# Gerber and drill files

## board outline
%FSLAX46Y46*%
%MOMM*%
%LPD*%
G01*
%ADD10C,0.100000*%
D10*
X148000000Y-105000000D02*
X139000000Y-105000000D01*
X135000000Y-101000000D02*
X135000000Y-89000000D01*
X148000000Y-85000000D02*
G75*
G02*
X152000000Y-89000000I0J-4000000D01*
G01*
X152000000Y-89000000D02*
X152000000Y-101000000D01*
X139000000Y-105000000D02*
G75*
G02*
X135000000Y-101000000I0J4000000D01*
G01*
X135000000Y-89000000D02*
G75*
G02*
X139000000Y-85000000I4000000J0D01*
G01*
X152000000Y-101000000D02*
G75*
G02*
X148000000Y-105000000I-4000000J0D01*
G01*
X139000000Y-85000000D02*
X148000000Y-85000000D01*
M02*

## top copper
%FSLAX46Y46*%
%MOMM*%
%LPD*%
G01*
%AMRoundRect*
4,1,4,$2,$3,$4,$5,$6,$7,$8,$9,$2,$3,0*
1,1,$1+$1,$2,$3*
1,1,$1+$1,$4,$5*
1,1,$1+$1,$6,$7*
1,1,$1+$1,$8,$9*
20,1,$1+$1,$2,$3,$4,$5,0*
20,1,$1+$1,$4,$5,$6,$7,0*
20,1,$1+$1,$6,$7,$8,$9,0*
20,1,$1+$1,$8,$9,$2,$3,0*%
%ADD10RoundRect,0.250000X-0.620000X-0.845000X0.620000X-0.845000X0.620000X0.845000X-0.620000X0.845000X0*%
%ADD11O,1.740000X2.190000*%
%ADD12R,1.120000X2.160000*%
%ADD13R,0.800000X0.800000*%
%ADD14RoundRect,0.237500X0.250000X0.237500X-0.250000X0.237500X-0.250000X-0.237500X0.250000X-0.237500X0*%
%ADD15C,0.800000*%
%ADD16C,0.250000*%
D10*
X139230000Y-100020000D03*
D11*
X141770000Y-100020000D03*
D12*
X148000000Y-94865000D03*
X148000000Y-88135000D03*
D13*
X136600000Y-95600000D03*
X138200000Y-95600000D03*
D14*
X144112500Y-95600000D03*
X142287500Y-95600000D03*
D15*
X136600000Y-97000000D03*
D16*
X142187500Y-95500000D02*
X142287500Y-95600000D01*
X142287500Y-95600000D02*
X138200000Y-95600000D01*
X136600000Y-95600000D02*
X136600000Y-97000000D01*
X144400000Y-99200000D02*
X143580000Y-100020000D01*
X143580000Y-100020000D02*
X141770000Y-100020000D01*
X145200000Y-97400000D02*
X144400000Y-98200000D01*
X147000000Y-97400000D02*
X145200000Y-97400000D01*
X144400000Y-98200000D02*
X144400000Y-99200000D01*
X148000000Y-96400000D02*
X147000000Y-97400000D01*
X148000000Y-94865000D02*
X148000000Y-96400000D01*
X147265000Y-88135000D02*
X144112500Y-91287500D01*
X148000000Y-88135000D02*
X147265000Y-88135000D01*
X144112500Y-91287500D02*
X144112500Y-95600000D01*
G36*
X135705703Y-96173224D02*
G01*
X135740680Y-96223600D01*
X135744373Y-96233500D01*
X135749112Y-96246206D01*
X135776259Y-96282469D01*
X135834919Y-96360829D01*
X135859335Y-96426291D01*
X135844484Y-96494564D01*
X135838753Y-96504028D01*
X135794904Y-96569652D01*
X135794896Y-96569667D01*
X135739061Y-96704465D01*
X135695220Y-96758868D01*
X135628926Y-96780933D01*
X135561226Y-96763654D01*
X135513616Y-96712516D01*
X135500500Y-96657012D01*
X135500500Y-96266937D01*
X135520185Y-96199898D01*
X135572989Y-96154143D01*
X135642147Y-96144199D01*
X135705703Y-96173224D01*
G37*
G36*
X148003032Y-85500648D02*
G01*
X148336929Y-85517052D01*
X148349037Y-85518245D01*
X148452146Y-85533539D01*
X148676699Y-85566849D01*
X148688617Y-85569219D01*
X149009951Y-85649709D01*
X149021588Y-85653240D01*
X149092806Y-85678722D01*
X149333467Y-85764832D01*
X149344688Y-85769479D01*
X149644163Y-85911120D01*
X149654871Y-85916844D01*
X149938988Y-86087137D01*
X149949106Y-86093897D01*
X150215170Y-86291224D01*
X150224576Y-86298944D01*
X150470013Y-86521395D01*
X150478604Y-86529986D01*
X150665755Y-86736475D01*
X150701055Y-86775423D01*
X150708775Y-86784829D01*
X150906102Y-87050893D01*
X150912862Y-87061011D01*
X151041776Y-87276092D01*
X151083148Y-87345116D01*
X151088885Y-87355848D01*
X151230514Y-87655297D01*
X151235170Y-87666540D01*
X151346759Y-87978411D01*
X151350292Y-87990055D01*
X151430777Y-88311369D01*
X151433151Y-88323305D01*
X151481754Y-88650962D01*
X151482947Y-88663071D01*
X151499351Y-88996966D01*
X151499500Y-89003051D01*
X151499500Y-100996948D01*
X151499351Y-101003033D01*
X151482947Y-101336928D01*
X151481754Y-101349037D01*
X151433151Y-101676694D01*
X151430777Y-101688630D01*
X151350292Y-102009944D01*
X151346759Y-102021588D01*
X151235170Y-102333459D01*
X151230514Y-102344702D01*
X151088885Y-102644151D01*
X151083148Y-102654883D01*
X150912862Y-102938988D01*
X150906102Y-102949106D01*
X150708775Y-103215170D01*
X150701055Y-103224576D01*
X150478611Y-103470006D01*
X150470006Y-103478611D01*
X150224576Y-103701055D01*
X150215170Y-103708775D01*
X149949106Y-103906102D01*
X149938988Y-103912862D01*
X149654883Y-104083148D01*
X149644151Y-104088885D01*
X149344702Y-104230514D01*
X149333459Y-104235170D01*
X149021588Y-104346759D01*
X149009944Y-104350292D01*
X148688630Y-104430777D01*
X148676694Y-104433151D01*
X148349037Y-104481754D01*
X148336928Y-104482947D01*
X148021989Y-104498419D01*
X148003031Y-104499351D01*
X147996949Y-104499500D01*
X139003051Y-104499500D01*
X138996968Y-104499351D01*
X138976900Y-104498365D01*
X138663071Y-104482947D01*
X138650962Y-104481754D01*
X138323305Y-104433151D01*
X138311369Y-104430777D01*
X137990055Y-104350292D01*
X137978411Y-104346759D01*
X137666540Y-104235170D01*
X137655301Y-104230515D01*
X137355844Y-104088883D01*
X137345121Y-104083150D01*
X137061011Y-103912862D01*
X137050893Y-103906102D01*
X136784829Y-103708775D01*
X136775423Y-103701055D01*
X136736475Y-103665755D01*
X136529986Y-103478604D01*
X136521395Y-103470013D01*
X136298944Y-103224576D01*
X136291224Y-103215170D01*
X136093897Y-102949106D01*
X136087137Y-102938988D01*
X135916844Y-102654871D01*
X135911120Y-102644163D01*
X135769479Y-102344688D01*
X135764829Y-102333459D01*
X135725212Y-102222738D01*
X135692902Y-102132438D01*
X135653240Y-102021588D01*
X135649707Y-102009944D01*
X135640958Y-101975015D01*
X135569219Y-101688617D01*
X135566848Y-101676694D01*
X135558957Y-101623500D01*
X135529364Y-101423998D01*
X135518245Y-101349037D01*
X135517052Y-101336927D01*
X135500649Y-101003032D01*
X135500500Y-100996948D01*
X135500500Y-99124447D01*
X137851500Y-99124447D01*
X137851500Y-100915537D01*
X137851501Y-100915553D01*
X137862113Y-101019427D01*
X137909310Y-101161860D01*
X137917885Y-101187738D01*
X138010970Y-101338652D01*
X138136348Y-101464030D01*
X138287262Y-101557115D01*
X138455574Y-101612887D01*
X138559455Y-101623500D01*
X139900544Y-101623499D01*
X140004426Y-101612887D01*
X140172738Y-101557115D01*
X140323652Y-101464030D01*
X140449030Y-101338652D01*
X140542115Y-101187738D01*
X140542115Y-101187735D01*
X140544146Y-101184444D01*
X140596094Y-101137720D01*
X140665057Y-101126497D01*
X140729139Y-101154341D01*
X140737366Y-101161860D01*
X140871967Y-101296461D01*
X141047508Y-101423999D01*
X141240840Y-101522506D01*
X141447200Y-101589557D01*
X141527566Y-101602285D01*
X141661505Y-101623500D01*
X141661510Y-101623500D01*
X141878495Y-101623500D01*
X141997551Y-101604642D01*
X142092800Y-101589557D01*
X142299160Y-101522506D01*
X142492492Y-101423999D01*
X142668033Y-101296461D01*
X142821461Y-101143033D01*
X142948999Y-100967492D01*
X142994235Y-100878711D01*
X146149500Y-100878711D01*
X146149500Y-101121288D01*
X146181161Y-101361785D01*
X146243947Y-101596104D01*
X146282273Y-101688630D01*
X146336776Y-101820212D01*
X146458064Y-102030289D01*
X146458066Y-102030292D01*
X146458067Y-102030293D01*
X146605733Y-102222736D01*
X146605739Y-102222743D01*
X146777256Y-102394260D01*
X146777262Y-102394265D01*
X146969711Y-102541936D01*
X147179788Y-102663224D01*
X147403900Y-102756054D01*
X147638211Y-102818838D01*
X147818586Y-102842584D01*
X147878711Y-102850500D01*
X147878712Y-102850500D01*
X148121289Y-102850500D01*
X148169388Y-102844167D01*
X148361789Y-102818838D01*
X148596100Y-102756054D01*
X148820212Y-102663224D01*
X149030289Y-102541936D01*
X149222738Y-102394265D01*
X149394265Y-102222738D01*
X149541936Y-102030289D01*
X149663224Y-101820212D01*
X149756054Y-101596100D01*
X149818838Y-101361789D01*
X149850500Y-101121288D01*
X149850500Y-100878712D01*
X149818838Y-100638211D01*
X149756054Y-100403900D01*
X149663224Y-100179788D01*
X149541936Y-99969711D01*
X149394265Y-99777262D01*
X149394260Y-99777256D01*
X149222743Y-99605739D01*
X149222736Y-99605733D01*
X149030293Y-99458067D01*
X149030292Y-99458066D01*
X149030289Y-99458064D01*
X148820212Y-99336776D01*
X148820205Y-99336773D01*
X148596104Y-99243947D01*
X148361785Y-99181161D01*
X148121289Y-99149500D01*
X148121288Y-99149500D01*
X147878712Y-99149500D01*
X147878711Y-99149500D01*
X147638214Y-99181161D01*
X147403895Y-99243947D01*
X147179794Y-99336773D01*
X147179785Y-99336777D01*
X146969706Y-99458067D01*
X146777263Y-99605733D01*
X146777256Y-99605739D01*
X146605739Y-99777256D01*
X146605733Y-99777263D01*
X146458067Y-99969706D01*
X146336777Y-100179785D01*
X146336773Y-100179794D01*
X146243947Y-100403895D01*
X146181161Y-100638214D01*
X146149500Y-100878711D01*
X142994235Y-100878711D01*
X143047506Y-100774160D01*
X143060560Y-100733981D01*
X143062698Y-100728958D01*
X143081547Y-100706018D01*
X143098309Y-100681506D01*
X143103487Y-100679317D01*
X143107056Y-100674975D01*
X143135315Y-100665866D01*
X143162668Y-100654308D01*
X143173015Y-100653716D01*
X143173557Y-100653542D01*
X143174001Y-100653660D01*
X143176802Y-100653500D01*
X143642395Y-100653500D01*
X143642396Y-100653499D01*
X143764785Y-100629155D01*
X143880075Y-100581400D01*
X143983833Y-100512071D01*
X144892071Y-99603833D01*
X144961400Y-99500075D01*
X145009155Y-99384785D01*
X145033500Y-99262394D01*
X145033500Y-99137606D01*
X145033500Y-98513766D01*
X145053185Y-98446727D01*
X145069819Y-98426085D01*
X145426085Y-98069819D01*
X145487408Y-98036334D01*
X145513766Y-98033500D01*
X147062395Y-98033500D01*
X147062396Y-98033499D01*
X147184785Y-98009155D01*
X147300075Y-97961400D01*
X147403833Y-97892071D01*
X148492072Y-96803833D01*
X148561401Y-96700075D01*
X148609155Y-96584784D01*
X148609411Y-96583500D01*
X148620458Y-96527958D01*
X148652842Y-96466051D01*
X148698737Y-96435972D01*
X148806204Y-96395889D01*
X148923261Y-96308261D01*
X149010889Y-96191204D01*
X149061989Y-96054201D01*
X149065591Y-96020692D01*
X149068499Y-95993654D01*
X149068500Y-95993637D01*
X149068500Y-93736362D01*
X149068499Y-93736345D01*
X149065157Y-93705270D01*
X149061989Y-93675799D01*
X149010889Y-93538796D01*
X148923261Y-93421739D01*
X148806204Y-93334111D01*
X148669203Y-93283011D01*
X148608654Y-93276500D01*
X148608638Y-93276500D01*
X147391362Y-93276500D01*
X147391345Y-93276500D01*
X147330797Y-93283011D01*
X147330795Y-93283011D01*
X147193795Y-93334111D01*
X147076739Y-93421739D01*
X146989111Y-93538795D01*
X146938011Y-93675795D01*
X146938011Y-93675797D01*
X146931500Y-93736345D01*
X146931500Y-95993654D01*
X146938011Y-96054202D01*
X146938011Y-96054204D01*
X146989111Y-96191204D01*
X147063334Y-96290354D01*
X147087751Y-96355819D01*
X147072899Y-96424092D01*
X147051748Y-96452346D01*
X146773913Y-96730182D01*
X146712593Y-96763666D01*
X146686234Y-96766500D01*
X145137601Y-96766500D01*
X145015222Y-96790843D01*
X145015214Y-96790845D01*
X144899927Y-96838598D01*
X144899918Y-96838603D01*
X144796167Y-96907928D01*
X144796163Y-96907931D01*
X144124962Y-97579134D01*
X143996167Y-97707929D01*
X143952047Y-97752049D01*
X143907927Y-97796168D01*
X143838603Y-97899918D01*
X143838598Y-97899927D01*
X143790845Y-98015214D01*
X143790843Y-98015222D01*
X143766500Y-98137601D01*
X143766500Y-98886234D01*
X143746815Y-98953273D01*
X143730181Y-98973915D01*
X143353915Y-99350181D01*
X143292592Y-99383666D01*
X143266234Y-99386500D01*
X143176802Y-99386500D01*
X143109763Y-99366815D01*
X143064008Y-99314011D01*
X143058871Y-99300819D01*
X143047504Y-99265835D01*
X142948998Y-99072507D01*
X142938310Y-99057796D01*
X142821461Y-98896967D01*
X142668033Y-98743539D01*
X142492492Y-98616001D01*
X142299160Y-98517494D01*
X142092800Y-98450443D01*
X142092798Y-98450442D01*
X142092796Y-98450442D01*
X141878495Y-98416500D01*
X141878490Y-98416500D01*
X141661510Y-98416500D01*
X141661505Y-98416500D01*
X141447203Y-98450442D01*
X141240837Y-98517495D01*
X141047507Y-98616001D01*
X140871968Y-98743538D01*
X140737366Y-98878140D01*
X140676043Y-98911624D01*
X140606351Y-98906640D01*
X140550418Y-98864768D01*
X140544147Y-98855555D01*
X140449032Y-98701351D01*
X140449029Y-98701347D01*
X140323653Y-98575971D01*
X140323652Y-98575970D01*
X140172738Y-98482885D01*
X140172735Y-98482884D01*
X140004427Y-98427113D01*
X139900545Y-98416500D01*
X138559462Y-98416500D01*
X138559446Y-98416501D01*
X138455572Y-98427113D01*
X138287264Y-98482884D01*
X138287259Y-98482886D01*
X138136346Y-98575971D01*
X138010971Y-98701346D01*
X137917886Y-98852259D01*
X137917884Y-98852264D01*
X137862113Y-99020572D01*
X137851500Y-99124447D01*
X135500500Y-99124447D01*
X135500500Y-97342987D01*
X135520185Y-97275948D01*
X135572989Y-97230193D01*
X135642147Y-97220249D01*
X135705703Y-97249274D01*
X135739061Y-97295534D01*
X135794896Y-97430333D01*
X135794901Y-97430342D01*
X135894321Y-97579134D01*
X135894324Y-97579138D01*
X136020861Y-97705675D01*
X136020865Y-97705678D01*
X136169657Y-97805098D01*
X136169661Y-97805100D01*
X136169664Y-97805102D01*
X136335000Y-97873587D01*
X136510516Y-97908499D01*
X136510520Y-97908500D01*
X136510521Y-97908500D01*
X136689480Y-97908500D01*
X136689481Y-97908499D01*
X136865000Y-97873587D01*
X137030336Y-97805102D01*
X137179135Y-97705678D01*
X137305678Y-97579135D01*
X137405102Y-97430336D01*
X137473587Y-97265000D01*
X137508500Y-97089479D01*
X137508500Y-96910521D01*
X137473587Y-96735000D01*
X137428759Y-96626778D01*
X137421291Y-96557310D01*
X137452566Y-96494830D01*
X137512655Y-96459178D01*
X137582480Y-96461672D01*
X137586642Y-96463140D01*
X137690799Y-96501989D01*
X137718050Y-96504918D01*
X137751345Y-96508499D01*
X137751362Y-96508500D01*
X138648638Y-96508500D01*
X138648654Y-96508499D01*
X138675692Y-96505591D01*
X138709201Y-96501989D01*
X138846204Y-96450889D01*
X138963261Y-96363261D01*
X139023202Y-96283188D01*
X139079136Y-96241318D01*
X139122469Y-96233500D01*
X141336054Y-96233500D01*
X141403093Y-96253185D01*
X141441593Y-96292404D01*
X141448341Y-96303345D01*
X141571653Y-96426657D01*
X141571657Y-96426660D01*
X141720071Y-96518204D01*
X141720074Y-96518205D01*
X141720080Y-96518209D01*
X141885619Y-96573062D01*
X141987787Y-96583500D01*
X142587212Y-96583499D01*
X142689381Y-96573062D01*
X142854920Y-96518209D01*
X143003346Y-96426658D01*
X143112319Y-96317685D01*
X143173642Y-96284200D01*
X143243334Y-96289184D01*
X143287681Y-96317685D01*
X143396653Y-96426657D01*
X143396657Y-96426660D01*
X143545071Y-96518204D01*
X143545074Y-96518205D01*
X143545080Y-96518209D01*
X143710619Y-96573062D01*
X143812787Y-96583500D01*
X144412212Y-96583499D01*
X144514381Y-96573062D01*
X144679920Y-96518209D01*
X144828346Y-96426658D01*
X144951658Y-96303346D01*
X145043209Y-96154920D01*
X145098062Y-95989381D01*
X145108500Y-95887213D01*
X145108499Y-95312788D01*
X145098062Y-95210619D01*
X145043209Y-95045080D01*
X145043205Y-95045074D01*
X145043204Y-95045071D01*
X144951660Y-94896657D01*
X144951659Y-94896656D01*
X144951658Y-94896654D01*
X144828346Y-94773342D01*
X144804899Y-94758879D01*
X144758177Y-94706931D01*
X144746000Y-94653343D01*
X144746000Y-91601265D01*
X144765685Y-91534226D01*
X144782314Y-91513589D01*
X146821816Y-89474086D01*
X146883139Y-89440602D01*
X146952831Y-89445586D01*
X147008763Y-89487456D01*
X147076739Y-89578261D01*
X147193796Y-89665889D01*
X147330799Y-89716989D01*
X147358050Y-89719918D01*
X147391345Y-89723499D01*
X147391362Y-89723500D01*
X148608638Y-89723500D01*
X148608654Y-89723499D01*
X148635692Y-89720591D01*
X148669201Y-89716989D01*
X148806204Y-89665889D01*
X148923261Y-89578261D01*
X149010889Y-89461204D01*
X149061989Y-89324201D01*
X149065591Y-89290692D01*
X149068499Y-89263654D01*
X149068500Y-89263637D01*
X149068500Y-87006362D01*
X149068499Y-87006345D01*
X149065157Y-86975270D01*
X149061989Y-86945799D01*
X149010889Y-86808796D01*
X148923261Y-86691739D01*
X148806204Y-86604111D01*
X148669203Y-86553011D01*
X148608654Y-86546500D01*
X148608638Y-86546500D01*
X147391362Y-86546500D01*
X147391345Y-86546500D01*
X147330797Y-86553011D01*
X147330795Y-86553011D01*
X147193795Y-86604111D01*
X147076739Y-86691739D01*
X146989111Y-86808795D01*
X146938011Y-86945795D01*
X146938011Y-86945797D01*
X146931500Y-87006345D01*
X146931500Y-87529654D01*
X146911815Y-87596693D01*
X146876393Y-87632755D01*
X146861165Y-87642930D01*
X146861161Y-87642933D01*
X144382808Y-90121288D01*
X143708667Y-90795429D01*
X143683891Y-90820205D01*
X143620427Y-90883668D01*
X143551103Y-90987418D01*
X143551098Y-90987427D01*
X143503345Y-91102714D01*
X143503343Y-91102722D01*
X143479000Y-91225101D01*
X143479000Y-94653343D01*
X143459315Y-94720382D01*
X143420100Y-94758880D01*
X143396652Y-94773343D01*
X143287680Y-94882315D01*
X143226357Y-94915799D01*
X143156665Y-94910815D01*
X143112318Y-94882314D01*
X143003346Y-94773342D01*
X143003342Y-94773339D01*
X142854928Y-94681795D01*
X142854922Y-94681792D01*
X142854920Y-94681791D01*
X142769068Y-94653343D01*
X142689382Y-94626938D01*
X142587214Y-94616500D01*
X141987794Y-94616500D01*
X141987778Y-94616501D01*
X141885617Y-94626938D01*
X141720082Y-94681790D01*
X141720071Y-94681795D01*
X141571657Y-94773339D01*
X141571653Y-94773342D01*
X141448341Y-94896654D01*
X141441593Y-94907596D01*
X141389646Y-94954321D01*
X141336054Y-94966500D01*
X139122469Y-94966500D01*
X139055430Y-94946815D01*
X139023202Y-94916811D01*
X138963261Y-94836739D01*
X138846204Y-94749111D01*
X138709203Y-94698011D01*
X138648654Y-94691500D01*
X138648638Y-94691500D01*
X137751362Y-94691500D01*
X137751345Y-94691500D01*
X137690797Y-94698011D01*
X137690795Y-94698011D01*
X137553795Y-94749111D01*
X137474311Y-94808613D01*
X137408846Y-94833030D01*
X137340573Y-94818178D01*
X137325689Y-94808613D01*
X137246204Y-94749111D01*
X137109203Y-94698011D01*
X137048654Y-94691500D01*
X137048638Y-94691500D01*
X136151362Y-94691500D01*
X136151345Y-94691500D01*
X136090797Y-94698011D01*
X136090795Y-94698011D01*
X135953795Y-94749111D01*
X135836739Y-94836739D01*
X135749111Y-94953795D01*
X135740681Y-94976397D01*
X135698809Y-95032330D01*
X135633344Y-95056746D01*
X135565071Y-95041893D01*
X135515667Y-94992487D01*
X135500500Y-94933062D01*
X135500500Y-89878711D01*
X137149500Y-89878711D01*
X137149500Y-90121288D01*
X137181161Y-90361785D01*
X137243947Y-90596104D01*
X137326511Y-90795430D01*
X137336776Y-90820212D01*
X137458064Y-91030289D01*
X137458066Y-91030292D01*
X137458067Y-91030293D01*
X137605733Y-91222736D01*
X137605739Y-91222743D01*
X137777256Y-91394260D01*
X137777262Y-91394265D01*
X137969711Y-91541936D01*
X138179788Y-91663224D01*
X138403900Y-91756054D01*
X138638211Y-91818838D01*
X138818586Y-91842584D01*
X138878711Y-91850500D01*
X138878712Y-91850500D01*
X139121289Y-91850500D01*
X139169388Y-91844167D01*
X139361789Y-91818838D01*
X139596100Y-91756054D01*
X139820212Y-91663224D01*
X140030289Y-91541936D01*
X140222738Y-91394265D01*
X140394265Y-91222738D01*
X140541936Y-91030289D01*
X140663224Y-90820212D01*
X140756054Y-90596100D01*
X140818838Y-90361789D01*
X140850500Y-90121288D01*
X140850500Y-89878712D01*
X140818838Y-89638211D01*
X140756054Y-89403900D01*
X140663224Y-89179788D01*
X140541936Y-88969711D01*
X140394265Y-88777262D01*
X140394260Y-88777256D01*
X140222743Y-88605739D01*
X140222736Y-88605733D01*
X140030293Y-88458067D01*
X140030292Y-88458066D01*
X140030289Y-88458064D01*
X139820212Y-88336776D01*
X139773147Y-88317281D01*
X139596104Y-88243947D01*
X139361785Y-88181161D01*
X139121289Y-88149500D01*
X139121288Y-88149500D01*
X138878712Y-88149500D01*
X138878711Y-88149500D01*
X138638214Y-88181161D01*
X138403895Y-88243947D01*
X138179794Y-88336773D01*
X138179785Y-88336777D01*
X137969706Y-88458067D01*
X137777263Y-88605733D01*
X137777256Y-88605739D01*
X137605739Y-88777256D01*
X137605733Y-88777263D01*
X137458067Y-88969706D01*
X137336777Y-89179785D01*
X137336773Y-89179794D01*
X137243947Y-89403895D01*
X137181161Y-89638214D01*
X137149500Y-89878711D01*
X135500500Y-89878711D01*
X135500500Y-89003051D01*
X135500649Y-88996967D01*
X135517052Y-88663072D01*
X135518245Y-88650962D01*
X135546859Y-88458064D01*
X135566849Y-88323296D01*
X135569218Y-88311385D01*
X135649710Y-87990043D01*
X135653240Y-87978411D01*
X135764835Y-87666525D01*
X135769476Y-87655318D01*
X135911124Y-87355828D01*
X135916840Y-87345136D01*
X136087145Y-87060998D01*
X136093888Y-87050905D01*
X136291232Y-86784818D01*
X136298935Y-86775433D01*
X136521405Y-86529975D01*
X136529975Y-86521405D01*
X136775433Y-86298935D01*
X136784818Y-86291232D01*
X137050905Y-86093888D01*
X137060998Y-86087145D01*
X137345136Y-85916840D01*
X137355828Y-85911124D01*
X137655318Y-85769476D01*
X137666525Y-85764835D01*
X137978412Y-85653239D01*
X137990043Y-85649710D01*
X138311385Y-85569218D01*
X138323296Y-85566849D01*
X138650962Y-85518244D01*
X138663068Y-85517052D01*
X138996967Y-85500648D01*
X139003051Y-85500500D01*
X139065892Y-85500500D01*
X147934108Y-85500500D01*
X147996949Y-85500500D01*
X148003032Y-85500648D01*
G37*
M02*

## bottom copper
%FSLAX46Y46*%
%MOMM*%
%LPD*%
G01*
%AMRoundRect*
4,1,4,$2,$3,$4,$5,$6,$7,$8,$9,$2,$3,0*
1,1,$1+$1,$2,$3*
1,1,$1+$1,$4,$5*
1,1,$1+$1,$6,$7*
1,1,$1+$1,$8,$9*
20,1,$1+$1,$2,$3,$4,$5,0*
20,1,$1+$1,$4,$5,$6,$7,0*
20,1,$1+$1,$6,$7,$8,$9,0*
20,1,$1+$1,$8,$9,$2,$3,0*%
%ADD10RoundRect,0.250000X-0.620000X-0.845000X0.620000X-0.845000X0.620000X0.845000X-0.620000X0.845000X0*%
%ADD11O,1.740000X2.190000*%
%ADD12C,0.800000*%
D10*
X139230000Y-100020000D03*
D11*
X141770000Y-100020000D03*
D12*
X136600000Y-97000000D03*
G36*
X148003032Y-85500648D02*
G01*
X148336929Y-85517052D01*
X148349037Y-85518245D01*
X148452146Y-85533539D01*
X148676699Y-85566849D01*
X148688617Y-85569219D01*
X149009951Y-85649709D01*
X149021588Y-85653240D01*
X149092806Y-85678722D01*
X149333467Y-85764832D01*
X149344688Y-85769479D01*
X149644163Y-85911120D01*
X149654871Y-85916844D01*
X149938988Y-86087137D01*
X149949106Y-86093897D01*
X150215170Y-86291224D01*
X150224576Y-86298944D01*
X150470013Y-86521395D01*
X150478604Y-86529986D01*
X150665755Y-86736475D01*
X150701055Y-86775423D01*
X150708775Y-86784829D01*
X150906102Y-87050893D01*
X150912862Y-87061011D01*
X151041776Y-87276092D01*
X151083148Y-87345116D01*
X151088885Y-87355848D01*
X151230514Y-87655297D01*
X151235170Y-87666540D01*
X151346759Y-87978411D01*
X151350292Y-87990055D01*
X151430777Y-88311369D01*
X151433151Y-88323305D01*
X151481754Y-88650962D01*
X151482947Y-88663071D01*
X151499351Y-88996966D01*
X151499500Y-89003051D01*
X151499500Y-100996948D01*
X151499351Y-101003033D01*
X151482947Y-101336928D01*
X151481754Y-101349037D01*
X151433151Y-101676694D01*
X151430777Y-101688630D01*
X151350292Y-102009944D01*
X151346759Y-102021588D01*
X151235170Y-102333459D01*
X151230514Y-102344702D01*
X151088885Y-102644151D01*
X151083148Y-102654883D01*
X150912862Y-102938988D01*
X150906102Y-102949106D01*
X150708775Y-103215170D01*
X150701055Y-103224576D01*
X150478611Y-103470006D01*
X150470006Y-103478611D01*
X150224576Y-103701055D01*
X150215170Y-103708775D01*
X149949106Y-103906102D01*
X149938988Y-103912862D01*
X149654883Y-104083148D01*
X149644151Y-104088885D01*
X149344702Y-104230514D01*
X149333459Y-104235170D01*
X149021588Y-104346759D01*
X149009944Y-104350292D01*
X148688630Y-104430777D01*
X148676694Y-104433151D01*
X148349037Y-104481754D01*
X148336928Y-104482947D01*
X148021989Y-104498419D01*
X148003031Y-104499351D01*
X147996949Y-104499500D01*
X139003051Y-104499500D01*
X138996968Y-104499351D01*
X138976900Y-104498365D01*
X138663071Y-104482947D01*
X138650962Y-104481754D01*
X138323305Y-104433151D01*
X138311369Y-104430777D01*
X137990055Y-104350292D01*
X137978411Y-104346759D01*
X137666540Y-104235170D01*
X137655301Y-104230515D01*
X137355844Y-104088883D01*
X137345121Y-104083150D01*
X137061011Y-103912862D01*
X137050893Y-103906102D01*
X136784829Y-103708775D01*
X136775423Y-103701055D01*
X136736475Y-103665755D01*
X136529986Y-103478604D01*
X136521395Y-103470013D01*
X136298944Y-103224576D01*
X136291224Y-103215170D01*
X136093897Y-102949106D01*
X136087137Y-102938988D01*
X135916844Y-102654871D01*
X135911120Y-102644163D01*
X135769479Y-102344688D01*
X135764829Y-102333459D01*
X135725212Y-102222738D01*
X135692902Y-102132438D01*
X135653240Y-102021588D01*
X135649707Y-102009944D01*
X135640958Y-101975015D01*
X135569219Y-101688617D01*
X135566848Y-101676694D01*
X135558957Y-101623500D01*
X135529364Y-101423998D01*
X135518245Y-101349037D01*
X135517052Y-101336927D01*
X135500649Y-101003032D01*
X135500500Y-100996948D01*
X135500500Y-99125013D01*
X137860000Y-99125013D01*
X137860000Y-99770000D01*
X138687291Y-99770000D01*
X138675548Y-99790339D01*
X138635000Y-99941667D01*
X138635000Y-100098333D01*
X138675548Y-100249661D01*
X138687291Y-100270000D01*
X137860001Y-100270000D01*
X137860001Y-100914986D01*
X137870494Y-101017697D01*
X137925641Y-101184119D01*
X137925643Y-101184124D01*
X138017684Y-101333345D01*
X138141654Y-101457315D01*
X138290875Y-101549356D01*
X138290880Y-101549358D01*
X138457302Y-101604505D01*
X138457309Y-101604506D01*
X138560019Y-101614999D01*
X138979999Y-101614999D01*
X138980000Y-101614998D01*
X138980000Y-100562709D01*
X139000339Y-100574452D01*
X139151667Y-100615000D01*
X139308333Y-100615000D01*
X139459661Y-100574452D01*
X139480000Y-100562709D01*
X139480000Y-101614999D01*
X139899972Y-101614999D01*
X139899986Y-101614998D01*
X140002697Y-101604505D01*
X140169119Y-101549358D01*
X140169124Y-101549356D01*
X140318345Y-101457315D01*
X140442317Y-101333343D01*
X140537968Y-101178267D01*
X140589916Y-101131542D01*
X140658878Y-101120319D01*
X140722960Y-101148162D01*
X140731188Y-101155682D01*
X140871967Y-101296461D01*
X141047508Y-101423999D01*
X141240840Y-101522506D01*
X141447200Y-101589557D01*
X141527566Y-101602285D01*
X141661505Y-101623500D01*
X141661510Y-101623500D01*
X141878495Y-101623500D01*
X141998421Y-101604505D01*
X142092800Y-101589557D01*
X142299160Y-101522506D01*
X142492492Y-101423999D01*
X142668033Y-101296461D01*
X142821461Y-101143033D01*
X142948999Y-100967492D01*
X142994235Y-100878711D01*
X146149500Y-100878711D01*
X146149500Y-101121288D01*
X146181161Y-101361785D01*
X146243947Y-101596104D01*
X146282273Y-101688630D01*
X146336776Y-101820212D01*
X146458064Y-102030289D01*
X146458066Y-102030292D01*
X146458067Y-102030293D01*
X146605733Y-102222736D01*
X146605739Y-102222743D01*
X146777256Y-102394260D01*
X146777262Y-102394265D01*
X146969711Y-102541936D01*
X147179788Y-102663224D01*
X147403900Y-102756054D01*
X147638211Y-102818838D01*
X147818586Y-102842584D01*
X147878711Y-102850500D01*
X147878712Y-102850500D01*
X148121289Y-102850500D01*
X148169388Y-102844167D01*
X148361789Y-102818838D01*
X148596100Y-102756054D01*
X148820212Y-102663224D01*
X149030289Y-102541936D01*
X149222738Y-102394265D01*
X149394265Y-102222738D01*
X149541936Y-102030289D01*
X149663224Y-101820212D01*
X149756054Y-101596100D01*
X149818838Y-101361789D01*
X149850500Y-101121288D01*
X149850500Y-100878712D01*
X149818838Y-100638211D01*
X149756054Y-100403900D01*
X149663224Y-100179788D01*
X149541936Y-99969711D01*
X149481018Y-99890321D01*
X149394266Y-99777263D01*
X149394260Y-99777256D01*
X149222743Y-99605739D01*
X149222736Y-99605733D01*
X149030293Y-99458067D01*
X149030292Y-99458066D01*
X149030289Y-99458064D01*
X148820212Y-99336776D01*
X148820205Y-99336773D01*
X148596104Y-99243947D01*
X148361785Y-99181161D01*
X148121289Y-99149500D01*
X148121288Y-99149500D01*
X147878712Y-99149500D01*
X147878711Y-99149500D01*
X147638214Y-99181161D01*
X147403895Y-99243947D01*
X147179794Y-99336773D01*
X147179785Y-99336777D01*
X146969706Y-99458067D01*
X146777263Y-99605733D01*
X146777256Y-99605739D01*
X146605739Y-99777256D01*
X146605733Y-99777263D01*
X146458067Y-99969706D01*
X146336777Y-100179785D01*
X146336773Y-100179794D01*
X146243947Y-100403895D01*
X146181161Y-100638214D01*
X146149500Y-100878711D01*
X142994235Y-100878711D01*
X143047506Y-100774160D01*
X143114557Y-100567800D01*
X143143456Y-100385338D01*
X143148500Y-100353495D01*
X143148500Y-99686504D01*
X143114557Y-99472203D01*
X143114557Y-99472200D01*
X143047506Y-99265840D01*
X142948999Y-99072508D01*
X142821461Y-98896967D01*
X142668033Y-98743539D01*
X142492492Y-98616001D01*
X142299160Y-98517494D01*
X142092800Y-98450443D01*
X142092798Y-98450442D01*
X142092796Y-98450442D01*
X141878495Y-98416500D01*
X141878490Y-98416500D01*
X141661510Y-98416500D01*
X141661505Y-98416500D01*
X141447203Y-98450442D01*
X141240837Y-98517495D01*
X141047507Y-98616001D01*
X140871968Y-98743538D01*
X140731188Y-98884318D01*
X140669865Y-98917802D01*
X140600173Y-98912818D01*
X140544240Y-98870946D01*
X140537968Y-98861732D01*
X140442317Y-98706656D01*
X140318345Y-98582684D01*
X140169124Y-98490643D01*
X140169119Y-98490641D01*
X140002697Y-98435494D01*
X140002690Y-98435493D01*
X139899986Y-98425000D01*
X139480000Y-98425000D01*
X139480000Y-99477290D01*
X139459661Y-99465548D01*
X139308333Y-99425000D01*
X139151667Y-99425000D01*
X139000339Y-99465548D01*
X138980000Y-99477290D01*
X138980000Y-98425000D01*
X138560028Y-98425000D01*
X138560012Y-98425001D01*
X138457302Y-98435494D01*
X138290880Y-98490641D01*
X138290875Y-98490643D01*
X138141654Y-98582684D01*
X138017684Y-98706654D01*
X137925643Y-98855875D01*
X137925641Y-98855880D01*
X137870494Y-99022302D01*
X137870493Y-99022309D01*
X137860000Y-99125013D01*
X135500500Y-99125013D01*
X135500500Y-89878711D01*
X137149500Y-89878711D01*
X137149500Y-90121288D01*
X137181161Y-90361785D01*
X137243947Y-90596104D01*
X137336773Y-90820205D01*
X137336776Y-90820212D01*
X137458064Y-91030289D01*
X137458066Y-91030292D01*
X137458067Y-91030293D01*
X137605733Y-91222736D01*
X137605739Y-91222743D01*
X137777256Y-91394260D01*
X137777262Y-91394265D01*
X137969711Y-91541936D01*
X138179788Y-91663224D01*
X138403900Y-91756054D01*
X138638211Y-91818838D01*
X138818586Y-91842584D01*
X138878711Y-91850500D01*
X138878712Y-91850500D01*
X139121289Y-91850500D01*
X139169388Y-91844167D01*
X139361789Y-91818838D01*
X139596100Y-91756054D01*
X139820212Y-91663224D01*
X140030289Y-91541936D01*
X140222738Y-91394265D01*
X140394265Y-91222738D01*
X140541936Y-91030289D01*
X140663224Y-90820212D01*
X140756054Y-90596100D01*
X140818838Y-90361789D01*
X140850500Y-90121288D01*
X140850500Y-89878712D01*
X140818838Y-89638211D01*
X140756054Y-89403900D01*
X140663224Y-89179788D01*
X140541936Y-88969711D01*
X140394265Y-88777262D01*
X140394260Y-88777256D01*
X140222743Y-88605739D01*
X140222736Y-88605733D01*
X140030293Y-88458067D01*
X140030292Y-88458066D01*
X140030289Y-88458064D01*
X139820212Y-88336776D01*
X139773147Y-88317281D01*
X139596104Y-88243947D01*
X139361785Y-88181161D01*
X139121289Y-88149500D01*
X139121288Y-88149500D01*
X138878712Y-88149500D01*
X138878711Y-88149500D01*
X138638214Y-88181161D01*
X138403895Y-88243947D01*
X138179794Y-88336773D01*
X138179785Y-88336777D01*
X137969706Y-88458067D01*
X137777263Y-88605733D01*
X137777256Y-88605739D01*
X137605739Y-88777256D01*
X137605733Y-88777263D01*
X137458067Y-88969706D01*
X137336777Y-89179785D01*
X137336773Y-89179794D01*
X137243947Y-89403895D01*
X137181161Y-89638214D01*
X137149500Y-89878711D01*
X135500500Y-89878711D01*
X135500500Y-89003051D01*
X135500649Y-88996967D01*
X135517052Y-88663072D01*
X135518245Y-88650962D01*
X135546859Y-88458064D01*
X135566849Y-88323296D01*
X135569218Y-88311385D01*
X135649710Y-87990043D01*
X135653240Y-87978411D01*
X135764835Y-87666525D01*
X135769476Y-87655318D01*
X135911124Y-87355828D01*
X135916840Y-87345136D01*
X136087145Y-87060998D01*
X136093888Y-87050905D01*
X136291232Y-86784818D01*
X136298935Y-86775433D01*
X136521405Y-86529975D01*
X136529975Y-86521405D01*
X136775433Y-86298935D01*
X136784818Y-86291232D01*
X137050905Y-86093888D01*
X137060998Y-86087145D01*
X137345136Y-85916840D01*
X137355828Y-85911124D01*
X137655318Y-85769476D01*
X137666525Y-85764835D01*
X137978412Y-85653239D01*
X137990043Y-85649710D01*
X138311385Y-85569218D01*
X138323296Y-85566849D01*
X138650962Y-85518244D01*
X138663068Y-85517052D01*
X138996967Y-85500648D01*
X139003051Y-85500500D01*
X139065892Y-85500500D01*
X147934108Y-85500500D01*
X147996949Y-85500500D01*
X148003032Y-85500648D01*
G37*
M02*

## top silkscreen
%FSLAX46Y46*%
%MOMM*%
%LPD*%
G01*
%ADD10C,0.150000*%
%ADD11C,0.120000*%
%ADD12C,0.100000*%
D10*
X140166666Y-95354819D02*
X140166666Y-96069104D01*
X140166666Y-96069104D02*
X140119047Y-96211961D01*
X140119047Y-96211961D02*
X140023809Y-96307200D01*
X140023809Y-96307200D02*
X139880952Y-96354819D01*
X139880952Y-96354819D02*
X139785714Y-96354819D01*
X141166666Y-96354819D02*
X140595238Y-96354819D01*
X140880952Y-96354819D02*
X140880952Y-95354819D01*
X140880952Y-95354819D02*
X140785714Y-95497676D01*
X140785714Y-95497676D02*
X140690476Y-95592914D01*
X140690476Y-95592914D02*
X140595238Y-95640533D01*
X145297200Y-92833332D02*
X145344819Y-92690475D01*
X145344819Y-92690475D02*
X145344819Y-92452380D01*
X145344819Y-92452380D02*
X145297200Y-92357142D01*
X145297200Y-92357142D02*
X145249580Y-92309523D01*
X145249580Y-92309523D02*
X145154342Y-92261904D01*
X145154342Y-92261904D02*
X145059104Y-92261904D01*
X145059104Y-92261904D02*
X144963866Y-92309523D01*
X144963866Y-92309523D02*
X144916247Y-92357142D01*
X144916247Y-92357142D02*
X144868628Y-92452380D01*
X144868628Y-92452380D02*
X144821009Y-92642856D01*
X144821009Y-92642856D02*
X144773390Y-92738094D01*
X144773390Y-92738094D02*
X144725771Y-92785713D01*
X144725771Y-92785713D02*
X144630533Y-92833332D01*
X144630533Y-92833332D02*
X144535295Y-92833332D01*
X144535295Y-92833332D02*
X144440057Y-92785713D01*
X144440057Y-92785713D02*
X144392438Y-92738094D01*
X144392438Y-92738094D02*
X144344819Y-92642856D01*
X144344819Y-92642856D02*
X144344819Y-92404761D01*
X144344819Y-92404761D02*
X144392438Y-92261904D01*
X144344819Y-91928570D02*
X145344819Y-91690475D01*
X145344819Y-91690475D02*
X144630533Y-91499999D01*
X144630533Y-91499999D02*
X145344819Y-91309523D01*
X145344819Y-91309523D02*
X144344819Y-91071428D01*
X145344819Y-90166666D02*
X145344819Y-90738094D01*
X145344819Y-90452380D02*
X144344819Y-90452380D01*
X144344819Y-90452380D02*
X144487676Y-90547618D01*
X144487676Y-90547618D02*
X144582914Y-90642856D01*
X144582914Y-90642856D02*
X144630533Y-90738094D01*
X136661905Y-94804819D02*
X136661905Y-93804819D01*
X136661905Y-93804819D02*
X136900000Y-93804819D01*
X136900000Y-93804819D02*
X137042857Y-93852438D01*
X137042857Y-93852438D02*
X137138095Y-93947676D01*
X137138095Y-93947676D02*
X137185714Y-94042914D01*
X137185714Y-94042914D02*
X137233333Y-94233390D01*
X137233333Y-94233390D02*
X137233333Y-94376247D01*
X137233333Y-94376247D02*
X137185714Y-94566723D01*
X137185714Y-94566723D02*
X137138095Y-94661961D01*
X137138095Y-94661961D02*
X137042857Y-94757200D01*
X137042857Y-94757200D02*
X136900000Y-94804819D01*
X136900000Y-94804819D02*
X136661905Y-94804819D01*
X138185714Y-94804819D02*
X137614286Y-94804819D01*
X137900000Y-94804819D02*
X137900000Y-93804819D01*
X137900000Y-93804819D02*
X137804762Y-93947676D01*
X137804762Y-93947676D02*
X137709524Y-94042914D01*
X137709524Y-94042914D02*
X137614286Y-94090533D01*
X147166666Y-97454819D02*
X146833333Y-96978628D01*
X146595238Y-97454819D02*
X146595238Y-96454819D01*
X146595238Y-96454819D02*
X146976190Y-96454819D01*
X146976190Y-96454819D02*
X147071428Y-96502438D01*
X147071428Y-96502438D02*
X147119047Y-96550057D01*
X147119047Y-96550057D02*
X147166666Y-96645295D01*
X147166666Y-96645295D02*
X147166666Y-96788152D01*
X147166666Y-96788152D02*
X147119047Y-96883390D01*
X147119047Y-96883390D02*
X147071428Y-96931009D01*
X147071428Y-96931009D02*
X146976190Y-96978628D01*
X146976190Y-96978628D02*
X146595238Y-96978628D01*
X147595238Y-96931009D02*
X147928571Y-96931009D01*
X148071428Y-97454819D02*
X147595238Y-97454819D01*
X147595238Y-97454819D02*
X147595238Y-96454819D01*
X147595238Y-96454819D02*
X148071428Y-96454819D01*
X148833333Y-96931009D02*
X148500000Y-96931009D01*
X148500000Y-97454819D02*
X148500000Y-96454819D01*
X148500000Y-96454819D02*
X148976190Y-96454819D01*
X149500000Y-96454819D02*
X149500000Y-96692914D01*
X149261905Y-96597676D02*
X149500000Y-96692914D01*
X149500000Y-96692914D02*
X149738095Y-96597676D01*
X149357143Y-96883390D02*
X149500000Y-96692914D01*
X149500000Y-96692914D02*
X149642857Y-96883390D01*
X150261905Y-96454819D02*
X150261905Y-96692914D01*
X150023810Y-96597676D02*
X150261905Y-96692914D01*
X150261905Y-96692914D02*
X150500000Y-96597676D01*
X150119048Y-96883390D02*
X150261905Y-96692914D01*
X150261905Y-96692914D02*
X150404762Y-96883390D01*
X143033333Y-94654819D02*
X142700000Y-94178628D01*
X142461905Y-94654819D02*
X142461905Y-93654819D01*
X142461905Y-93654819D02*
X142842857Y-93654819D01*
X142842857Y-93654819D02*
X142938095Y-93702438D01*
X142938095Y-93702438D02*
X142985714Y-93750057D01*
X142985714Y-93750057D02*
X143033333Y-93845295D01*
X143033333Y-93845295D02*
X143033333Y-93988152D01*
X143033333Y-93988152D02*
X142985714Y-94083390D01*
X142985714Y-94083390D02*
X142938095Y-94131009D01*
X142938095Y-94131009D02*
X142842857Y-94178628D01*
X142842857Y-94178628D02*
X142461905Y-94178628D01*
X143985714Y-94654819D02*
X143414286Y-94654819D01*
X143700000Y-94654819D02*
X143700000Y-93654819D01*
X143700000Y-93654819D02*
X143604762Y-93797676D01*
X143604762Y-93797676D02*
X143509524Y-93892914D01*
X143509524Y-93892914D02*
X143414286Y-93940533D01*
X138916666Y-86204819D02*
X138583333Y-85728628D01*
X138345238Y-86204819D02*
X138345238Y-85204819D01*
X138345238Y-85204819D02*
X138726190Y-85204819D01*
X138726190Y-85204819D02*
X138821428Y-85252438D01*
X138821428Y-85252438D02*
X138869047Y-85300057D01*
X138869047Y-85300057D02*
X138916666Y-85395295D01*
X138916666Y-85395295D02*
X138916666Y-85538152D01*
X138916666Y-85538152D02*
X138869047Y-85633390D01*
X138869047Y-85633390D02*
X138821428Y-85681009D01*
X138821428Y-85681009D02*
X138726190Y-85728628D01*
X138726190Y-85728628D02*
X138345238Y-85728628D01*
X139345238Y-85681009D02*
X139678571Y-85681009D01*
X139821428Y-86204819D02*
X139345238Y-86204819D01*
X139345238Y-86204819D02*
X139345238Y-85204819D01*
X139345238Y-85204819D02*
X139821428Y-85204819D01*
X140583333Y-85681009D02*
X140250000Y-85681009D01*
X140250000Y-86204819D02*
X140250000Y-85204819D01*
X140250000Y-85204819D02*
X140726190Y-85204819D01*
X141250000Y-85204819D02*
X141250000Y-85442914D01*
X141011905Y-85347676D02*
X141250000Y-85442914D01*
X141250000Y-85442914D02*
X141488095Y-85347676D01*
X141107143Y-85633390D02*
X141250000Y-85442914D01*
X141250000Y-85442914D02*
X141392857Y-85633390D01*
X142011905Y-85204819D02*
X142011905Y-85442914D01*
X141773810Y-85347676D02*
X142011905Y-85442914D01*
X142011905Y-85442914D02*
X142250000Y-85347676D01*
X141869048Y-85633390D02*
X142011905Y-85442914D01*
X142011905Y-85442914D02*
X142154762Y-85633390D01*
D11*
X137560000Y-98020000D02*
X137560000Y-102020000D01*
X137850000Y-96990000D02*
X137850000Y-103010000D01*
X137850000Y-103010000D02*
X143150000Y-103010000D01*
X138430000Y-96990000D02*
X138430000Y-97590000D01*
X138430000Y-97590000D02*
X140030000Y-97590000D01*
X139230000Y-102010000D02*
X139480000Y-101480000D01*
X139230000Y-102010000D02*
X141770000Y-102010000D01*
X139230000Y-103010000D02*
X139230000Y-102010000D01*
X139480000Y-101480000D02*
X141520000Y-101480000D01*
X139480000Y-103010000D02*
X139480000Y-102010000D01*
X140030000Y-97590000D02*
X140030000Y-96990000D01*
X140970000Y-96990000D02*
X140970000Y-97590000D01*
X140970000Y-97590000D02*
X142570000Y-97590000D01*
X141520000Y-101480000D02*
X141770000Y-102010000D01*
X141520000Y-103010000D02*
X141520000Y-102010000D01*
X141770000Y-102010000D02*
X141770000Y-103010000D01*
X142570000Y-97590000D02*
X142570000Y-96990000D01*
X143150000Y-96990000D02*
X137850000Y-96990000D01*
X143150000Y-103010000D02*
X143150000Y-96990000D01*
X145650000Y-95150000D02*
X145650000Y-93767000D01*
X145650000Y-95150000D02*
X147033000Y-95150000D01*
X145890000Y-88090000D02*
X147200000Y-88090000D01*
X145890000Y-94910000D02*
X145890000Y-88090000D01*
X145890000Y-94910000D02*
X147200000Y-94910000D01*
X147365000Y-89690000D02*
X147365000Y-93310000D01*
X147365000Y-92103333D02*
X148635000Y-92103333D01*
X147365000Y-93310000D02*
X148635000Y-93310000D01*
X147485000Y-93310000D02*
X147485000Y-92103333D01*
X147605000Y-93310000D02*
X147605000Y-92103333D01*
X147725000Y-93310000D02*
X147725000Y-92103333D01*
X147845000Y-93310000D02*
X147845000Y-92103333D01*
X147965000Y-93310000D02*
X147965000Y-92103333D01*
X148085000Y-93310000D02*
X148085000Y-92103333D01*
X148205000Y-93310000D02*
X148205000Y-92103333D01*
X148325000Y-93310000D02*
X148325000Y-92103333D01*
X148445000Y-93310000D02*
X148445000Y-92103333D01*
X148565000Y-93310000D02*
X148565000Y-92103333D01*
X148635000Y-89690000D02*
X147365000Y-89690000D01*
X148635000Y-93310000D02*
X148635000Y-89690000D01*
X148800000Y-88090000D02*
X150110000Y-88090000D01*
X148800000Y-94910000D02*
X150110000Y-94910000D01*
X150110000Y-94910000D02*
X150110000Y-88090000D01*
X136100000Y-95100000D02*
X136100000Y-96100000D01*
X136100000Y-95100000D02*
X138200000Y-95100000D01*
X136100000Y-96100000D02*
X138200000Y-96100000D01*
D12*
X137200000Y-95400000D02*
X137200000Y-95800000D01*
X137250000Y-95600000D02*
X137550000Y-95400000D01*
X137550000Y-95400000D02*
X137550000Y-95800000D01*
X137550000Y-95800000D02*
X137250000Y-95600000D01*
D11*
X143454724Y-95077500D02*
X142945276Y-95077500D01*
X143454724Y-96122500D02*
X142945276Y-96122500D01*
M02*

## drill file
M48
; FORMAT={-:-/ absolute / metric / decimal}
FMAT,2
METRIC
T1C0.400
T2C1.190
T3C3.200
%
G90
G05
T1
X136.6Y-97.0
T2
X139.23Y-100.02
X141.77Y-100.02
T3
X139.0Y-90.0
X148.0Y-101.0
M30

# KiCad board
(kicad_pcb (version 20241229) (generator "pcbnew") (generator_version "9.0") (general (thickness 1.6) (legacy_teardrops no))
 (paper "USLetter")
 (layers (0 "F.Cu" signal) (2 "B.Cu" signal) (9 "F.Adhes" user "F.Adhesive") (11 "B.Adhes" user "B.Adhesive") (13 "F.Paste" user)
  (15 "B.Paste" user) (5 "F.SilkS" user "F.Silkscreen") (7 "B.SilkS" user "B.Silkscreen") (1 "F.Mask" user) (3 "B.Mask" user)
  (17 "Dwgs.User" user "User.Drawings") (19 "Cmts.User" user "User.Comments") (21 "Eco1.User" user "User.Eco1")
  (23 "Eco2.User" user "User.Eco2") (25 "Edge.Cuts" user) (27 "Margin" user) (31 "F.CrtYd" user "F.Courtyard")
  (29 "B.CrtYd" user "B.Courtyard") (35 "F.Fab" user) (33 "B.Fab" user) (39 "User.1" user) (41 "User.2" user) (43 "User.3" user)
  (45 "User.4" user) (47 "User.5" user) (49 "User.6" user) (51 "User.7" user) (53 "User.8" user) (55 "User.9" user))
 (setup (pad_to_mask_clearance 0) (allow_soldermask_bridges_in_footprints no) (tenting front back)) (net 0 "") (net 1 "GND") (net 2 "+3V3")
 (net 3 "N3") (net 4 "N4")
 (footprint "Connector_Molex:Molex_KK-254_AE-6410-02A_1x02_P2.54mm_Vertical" (layer "F.Cu") (at 139.23 100.02)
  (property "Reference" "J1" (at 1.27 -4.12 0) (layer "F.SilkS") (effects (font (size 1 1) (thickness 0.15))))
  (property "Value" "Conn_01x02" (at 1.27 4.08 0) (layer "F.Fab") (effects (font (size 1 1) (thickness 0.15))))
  (fp_line (start -1.67 -2) (end -1.67 2) (stroke (width 0.12) (type solid)) (layer "F.SilkS"))
  (fp_line (start -1.38 -3.03) (end -1.38 2.99) (stroke (width 0.12) (type solid)) (layer "F.SilkS"))
  (fp_line (start -1.38 2.99) (end 3.92 2.99) (stroke (width 0.12) (type solid)) (layer "F.SilkS"))
  (fp_line (start -0.8 -3.03) (end -0.8 -2.43) (stroke (width 0.12) (type solid)) (layer "F.SilkS"))
  (fp_line (start -0.8 -2.43) (end 0.8 -2.43) (stroke (width 0.12) (type solid)) (layer "F.SilkS"))
  (fp_line (start 0 1.99) (end 0.25 1.46) (stroke (width 0.12) (type solid)) (layer "F.SilkS"))
  (fp_line (start 0 1.99) (end 2.54 1.99) (stroke (width 0.12) (type solid)) (layer "F.SilkS"))
  (fp_line (start 0 2.99) (end 0 1.99) (stroke (width 0.12) (type solid)) (layer "F.SilkS"))
  (fp_line (start 0.25 1.46) (end 2.29 1.46) (stroke (width 0.12) (type solid)) (layer "F.SilkS"))
  (fp_line (start 0.25 2.99) (end 0.25 1.99) (stroke (width 0.12) (type solid)) (layer "F.SilkS"))
  (fp_line (start 0.8 -2.43) (end 0.8 -3.03) (stroke (width 0.12) (type solid)) (layer "F.SilkS"))
  (fp_line (start 1.74 -3.03) (end 1.74 -2.43) (stroke (width 0.12) (type solid)) (layer "F.SilkS"))
  (fp_line (start 1.74 -2.43) (end 3.34 -2.43) (stroke (width 0.12) (type solid)) (layer "F.SilkS"))
  (fp_line (start 2.29 1.46) (end 2.54 1.99) (stroke (width 0.12) (type solid)) (layer "F.SilkS"))
  (fp_line (start 2.29 2.99) (end 2.29 1.99) (stroke (width 0.12) (type solid)) (layer "F.SilkS"))
  (fp_line (start 2.54 1.99) (end 2.54 2.99) (stroke (width 0.12) (type solid)) (layer "F.SilkS"))
  (fp_line (start 3.34 -2.43) (end 3.34 -3.03) (stroke (width 0.12) (type solid)) (layer "F.SilkS"))
  (fp_line (start 3.92 -3.03) (end -1.38 -3.03) (stroke (width 0.12) (type solid)) (layer "F.SilkS"))
  (fp_line (start 3.92 2.99) (end 3.92 -3.03) (stroke (width 0.12) (type solid)) (layer "F.SilkS"))
  (pad "1" thru_hole roundrect (at 0 0) (size 1.74 2.19) (drill 1.19) (layers "*.Cu" "*.Mask") (remove_unused_layers no)
   (roundrect_rratio 0.143678) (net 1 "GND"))
  (pad "2" thru_hole oval (at 2.54 0) (size 1.74 2.19) (drill 1.19) (layers "*.Cu" "*.Mask") (remove_unused_layers no) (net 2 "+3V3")))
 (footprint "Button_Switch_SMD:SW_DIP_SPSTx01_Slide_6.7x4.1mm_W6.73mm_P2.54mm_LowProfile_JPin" (layer "F.Cu") (at 148 91.5 90)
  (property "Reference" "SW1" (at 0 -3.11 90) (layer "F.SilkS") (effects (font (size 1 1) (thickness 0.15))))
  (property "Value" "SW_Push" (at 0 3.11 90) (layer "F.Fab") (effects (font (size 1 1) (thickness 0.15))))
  (fp_line (start -3.65 -2.35) (end -2.267 -2.35) (stroke (width 0.12) (type solid)) (layer "F.SilkS"))
  (fp_line (start -3.65 -2.35) (end -3.65 -0.967) (stroke (width 0.12) (type solid)) (layer "F.SilkS"))
  (fp_line (start 3.41 -2.11) (end 3.41 -0.8) (stroke (width 0.12) (type solid)) (layer "F.SilkS"))
  (fp_line (start -3.41 -2.11) (end 3.41 -2.11) (stroke (width 0.12) (type solid)) (layer "F.SilkS"))
  (fp_line (start -3.41 -2.11) (end -3.41 -0.8) (stroke (width 0.12) (type solid)) (layer "F.SilkS"))
  (fp_line (start 1.81 -0.635) (end -1.81 -0.635) (stroke (width 0.12) (type solid)) (layer "F.SilkS"))
  (fp_line (start -0.603333 -0.635) (end -0.603333 0.635) (stroke (width 0.12) (type solid)) (layer "F.SilkS"))
  (fp_line (start -1.81 -0.635) (end -1.81 0.635) (stroke (width 0.12) (type solid)) (layer "F.SilkS"))
  (fp_line (start -1.81 -0.515) (end -0.603333 -0.515) (stroke (width 0.12) (type solid)) (layer "F.SilkS"))
  (fp_line (start -1.81 -0.395) (end -0.603333 -0.395) (stroke (width 0.12) (type solid)) (layer "F.SilkS"))
  (fp_line (start -1.81 -0.275) (end -0.603333 -0.275) (stroke (width 0.12) (type solid)) (layer "F.SilkS"))
  (fp_line (start -1.81 -0.155) (end -0.603333 -0.155) (stroke (width 0.12) (type solid)) (layer "F.SilkS"))
  (fp_line (start -1.81 -0.035) (end -0.603333 -0.035) (stroke (width 0.12) (type solid)) (layer "F.SilkS"))
  (fp_line (start -1.81 0.085) (end -0.603333 0.085) (stroke (width 0.12) (type solid)) (layer "F.SilkS"))
  (fp_line (start -1.81 0.205) (end -0.603333 0.205) (stroke (width 0.12) (type solid)) (layer "F.SilkS"))
  (fp_line (start -1.81 0.325) (end -0.603333 0.325) (stroke (width 0.12) (type solid)) (layer "F.SilkS"))
  (fp_line (start -1.81 0.445) (end -0.603333 0.445) (stroke (width 0.12) (type solid)) (layer "F.SilkS"))
  (fp_line (start -1.81 0.565) (end -0.603333 0.565) (stroke (width 0.12) (type solid)) (layer "F.SilkS"))
  (fp_line (start 1.81 0.635) (end 1.81 -0.635) (stroke (width 0.12) (type solid)) (layer "F.SilkS"))
  (fp_line (start -1.81 0.635) (end 1.81 0.635) (stroke (width 0.12) (type solid)) (layer "F.SilkS"))
  (fp_line (start 3.41 0.8) (end 3.41 2.11) (stroke (width 0.12) (type solid)) (layer "F.SilkS"))
  (fp_line (start -3.41 0.8) (end -3.41 2.11) (stroke (width 0.12) (type solid)) (layer "F.SilkS"))
  (fp_line (start -3.41 2.11) (end 3.41 2.11) (stroke (width 0.12) (type solid)) (layer "F.SilkS"))
  (pad "1" smd rect (at -3.365 0 90) (size 2.16 1.12) (layers "F.Cu" "F.Mask" "F.Paste") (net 2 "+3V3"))
  (pad "2" smd rect (at 3.365 0 90) (size 2.16 1.12) (layers "F.Cu" "F.Mask" "F.Paste") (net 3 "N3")))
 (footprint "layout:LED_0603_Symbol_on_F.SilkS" (layer "F.Cu") (at 137.4 95.6)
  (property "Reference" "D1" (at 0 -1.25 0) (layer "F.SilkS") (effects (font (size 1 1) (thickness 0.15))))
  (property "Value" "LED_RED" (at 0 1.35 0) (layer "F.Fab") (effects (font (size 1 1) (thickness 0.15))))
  (fp_line (start -1.3 -0.5) (end -1.3 0.5) (stroke (width 0.12) (type solid)) (layer "F.SilkS"))
  (fp_line (start -1.3 -0.5) (end 0.8 -0.5) (stroke (width 0.12) (type solid)) (layer "F.SilkS"))
  (fp_line (start -1.3 0.5) (end 0.8 0.5) (stroke (width 0.12) (type solid)) (layer "F.SilkS"))
  (fp_line (start -0.2 -0.2) (end -0.2 0.2) (stroke (width 0.1) (type solid)) (layer "F.SilkS"))
  (fp_line (start -0.15 0) (end 0.15 -0.2) (stroke (width 0.1) (type solid)) (layer "F.SilkS"))
  (fp_line (start 0.15 -0.2) (end 0.15 0.2) (stroke (width 0.1) (type solid)) (layer "F.SilkS"))
  (fp_line (start 0.15 0.2) (end -0.15 0) (stroke (width 0.1) (type solid)) (layer "F.SilkS"))
  (pad "1" smd rect (at -0.8 0 180) (size 0.8 0.8) (layers "F.Cu" "F.Mask" "F.Paste") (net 1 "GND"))
  (pad "2" smd rect (at 0.8 0 180) (size 0.8 0.8) (layers "F.Cu" "F.Mask" "F.Paste") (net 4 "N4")))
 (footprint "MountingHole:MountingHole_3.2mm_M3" (layer "F.Cu") (at 148 101)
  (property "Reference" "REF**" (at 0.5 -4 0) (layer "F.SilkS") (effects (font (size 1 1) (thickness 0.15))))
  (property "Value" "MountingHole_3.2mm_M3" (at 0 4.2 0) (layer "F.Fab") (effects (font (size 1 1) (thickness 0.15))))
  (pad "" np_thru_hole circle (at 0 0) (size 3.2 3.2) (drill 3.2) (layers "*.Cu" "*.Mask")))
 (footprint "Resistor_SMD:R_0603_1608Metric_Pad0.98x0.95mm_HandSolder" (layer "F.Cu") (at 143.2 95.6 180)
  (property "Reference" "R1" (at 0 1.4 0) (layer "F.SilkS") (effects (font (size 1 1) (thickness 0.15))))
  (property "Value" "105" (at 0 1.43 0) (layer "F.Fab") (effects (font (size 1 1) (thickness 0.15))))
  (fp_line (start -0.254724 0.5225) (end 0.254724 0.5225) (stroke (width 0.12) (type solid)) (layer "F.SilkS"))
  (fp_line (start -0.254724 -0.5225) (end 0.254724 -0.5225) (stroke (width 0.12) (type solid)) (layer "F.SilkS"))
  (pad "1" smd roundrect (at -0.9125 0 180) (size 0.975 0.95) (layers "F.Cu" "F.Mask" "F.Paste") (roundrect_rratio 0.25) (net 3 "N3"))
  (pad "2" smd roundrect (at 0.9125 0 180) (size 0.975 0.95) (layers "F.Cu" "F.Mask" "F.Paste") (roundrect_rratio 0.25) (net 4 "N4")))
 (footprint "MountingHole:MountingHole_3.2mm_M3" (layer "F.Cu") (at 139 90)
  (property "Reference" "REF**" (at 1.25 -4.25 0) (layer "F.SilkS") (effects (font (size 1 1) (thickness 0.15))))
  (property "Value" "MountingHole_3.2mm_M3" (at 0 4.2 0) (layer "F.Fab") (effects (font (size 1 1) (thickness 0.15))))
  (pad "" np_thru_hole circle (at 0 0) (size 3.2 3.2) (drill 3.2) (layers "*.Cu" "*.Mask")))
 (gr_line (start 148 105) (end 139 105) (stroke (width 0.1) (type default)) (layer "Edge.Cuts"))
 (gr_line (start 135 101) (end 135 89) (stroke (width 0.1) (type default)) (layer "Edge.Cuts"))
 (gr_arc (start 148 85) (mid 150.828427 86.171573) (end 152 89) (stroke (width 0.1) (type default)) (layer "Edge.Cuts"))
 (gr_line (start 152 89) (end 152 101) (stroke (width 0.1) (type default)) (layer "Edge.Cuts"))
 (gr_arc (start 139 105) (mid 136.171573 103.828427) (end 135 101) (stroke (width 0.1) (type default)) (layer "Edge.Cuts"))
 (gr_arc (start 135 89) (mid 136.171573 86.171573) (end 139 85) (stroke (width 0.1) (type default)) (layer "Edge.Cuts"))
 (gr_arc (start 152 101) (mid 150.828427 103.828427) (end 148 105) (stroke (width 0.1) (type default)) (layer "Edge.Cuts"))
 (gr_line (start 139 85) (end 148 85) (stroke (width 0.1) (type default)) (layer "Edge.Cuts"))
 (segment (start 142.1875 95.5) (end 142.2875 95.6) (width 0.25) (layer "F.Cu") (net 4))
 (segment (start 142.2875 95.6) (end 138.2 95.6) (width 0.25) (layer "F.Cu") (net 4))
 (segment (start 136.6 95.6) (end 136.6 97) (width 0.25) (layer "F.Cu") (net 1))
 (via (at 136.6 97) (size 0.8) (drill 0.4) (layers "F.Cu" "B.Cu") (free yes) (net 1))
 (segment (start 144.4 99.2) (end 143.58 100.02) (width 0.25) (layer "F.Cu") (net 2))
 (segment (start 143.58 100.02) (end 141.77 100.02) (width 0.25) (layer "F.Cu") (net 2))
 (segment (start 145.2 97.4) (end 144.4 98.2) (width 0.25) (layer "F.Cu") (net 2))
 (segment (start 147 97.4) (end 145.2 97.4) (width 0.25) (layer "F.Cu") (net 2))
 (segment (start 144.4 98.2) (end 144.4 99.2) (width 0.25) (layer "F.Cu") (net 2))
 (segment (start 148 96.4) (end 147 97.4) (width 0.25) (layer "F.Cu") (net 2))
 (segment (start 148 94.865) (end 148 96.4) (width 0.25) (layer "F.Cu") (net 2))
 (segment (start 147.265 88.135) (end 144.1125 91.2875) (width 0.25) (layer "F.Cu") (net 3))
 (segment (start 148 88.135) (end 147.265 88.135) (width 0.25) (layer "F.Cu") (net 3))
 (segment (start 144.1125 91.2875) (end 144.1125 95.6) (width 0.25) (layer "F.Cu") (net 3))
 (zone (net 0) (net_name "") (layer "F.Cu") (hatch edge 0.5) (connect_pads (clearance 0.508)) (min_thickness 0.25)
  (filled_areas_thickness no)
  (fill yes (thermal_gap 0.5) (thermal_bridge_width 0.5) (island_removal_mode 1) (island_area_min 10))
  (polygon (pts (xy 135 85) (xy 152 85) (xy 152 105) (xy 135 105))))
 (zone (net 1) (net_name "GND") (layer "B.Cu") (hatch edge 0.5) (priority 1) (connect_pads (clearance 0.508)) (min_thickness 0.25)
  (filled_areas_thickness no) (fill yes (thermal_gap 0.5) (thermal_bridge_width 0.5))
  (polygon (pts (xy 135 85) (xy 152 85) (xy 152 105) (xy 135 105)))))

